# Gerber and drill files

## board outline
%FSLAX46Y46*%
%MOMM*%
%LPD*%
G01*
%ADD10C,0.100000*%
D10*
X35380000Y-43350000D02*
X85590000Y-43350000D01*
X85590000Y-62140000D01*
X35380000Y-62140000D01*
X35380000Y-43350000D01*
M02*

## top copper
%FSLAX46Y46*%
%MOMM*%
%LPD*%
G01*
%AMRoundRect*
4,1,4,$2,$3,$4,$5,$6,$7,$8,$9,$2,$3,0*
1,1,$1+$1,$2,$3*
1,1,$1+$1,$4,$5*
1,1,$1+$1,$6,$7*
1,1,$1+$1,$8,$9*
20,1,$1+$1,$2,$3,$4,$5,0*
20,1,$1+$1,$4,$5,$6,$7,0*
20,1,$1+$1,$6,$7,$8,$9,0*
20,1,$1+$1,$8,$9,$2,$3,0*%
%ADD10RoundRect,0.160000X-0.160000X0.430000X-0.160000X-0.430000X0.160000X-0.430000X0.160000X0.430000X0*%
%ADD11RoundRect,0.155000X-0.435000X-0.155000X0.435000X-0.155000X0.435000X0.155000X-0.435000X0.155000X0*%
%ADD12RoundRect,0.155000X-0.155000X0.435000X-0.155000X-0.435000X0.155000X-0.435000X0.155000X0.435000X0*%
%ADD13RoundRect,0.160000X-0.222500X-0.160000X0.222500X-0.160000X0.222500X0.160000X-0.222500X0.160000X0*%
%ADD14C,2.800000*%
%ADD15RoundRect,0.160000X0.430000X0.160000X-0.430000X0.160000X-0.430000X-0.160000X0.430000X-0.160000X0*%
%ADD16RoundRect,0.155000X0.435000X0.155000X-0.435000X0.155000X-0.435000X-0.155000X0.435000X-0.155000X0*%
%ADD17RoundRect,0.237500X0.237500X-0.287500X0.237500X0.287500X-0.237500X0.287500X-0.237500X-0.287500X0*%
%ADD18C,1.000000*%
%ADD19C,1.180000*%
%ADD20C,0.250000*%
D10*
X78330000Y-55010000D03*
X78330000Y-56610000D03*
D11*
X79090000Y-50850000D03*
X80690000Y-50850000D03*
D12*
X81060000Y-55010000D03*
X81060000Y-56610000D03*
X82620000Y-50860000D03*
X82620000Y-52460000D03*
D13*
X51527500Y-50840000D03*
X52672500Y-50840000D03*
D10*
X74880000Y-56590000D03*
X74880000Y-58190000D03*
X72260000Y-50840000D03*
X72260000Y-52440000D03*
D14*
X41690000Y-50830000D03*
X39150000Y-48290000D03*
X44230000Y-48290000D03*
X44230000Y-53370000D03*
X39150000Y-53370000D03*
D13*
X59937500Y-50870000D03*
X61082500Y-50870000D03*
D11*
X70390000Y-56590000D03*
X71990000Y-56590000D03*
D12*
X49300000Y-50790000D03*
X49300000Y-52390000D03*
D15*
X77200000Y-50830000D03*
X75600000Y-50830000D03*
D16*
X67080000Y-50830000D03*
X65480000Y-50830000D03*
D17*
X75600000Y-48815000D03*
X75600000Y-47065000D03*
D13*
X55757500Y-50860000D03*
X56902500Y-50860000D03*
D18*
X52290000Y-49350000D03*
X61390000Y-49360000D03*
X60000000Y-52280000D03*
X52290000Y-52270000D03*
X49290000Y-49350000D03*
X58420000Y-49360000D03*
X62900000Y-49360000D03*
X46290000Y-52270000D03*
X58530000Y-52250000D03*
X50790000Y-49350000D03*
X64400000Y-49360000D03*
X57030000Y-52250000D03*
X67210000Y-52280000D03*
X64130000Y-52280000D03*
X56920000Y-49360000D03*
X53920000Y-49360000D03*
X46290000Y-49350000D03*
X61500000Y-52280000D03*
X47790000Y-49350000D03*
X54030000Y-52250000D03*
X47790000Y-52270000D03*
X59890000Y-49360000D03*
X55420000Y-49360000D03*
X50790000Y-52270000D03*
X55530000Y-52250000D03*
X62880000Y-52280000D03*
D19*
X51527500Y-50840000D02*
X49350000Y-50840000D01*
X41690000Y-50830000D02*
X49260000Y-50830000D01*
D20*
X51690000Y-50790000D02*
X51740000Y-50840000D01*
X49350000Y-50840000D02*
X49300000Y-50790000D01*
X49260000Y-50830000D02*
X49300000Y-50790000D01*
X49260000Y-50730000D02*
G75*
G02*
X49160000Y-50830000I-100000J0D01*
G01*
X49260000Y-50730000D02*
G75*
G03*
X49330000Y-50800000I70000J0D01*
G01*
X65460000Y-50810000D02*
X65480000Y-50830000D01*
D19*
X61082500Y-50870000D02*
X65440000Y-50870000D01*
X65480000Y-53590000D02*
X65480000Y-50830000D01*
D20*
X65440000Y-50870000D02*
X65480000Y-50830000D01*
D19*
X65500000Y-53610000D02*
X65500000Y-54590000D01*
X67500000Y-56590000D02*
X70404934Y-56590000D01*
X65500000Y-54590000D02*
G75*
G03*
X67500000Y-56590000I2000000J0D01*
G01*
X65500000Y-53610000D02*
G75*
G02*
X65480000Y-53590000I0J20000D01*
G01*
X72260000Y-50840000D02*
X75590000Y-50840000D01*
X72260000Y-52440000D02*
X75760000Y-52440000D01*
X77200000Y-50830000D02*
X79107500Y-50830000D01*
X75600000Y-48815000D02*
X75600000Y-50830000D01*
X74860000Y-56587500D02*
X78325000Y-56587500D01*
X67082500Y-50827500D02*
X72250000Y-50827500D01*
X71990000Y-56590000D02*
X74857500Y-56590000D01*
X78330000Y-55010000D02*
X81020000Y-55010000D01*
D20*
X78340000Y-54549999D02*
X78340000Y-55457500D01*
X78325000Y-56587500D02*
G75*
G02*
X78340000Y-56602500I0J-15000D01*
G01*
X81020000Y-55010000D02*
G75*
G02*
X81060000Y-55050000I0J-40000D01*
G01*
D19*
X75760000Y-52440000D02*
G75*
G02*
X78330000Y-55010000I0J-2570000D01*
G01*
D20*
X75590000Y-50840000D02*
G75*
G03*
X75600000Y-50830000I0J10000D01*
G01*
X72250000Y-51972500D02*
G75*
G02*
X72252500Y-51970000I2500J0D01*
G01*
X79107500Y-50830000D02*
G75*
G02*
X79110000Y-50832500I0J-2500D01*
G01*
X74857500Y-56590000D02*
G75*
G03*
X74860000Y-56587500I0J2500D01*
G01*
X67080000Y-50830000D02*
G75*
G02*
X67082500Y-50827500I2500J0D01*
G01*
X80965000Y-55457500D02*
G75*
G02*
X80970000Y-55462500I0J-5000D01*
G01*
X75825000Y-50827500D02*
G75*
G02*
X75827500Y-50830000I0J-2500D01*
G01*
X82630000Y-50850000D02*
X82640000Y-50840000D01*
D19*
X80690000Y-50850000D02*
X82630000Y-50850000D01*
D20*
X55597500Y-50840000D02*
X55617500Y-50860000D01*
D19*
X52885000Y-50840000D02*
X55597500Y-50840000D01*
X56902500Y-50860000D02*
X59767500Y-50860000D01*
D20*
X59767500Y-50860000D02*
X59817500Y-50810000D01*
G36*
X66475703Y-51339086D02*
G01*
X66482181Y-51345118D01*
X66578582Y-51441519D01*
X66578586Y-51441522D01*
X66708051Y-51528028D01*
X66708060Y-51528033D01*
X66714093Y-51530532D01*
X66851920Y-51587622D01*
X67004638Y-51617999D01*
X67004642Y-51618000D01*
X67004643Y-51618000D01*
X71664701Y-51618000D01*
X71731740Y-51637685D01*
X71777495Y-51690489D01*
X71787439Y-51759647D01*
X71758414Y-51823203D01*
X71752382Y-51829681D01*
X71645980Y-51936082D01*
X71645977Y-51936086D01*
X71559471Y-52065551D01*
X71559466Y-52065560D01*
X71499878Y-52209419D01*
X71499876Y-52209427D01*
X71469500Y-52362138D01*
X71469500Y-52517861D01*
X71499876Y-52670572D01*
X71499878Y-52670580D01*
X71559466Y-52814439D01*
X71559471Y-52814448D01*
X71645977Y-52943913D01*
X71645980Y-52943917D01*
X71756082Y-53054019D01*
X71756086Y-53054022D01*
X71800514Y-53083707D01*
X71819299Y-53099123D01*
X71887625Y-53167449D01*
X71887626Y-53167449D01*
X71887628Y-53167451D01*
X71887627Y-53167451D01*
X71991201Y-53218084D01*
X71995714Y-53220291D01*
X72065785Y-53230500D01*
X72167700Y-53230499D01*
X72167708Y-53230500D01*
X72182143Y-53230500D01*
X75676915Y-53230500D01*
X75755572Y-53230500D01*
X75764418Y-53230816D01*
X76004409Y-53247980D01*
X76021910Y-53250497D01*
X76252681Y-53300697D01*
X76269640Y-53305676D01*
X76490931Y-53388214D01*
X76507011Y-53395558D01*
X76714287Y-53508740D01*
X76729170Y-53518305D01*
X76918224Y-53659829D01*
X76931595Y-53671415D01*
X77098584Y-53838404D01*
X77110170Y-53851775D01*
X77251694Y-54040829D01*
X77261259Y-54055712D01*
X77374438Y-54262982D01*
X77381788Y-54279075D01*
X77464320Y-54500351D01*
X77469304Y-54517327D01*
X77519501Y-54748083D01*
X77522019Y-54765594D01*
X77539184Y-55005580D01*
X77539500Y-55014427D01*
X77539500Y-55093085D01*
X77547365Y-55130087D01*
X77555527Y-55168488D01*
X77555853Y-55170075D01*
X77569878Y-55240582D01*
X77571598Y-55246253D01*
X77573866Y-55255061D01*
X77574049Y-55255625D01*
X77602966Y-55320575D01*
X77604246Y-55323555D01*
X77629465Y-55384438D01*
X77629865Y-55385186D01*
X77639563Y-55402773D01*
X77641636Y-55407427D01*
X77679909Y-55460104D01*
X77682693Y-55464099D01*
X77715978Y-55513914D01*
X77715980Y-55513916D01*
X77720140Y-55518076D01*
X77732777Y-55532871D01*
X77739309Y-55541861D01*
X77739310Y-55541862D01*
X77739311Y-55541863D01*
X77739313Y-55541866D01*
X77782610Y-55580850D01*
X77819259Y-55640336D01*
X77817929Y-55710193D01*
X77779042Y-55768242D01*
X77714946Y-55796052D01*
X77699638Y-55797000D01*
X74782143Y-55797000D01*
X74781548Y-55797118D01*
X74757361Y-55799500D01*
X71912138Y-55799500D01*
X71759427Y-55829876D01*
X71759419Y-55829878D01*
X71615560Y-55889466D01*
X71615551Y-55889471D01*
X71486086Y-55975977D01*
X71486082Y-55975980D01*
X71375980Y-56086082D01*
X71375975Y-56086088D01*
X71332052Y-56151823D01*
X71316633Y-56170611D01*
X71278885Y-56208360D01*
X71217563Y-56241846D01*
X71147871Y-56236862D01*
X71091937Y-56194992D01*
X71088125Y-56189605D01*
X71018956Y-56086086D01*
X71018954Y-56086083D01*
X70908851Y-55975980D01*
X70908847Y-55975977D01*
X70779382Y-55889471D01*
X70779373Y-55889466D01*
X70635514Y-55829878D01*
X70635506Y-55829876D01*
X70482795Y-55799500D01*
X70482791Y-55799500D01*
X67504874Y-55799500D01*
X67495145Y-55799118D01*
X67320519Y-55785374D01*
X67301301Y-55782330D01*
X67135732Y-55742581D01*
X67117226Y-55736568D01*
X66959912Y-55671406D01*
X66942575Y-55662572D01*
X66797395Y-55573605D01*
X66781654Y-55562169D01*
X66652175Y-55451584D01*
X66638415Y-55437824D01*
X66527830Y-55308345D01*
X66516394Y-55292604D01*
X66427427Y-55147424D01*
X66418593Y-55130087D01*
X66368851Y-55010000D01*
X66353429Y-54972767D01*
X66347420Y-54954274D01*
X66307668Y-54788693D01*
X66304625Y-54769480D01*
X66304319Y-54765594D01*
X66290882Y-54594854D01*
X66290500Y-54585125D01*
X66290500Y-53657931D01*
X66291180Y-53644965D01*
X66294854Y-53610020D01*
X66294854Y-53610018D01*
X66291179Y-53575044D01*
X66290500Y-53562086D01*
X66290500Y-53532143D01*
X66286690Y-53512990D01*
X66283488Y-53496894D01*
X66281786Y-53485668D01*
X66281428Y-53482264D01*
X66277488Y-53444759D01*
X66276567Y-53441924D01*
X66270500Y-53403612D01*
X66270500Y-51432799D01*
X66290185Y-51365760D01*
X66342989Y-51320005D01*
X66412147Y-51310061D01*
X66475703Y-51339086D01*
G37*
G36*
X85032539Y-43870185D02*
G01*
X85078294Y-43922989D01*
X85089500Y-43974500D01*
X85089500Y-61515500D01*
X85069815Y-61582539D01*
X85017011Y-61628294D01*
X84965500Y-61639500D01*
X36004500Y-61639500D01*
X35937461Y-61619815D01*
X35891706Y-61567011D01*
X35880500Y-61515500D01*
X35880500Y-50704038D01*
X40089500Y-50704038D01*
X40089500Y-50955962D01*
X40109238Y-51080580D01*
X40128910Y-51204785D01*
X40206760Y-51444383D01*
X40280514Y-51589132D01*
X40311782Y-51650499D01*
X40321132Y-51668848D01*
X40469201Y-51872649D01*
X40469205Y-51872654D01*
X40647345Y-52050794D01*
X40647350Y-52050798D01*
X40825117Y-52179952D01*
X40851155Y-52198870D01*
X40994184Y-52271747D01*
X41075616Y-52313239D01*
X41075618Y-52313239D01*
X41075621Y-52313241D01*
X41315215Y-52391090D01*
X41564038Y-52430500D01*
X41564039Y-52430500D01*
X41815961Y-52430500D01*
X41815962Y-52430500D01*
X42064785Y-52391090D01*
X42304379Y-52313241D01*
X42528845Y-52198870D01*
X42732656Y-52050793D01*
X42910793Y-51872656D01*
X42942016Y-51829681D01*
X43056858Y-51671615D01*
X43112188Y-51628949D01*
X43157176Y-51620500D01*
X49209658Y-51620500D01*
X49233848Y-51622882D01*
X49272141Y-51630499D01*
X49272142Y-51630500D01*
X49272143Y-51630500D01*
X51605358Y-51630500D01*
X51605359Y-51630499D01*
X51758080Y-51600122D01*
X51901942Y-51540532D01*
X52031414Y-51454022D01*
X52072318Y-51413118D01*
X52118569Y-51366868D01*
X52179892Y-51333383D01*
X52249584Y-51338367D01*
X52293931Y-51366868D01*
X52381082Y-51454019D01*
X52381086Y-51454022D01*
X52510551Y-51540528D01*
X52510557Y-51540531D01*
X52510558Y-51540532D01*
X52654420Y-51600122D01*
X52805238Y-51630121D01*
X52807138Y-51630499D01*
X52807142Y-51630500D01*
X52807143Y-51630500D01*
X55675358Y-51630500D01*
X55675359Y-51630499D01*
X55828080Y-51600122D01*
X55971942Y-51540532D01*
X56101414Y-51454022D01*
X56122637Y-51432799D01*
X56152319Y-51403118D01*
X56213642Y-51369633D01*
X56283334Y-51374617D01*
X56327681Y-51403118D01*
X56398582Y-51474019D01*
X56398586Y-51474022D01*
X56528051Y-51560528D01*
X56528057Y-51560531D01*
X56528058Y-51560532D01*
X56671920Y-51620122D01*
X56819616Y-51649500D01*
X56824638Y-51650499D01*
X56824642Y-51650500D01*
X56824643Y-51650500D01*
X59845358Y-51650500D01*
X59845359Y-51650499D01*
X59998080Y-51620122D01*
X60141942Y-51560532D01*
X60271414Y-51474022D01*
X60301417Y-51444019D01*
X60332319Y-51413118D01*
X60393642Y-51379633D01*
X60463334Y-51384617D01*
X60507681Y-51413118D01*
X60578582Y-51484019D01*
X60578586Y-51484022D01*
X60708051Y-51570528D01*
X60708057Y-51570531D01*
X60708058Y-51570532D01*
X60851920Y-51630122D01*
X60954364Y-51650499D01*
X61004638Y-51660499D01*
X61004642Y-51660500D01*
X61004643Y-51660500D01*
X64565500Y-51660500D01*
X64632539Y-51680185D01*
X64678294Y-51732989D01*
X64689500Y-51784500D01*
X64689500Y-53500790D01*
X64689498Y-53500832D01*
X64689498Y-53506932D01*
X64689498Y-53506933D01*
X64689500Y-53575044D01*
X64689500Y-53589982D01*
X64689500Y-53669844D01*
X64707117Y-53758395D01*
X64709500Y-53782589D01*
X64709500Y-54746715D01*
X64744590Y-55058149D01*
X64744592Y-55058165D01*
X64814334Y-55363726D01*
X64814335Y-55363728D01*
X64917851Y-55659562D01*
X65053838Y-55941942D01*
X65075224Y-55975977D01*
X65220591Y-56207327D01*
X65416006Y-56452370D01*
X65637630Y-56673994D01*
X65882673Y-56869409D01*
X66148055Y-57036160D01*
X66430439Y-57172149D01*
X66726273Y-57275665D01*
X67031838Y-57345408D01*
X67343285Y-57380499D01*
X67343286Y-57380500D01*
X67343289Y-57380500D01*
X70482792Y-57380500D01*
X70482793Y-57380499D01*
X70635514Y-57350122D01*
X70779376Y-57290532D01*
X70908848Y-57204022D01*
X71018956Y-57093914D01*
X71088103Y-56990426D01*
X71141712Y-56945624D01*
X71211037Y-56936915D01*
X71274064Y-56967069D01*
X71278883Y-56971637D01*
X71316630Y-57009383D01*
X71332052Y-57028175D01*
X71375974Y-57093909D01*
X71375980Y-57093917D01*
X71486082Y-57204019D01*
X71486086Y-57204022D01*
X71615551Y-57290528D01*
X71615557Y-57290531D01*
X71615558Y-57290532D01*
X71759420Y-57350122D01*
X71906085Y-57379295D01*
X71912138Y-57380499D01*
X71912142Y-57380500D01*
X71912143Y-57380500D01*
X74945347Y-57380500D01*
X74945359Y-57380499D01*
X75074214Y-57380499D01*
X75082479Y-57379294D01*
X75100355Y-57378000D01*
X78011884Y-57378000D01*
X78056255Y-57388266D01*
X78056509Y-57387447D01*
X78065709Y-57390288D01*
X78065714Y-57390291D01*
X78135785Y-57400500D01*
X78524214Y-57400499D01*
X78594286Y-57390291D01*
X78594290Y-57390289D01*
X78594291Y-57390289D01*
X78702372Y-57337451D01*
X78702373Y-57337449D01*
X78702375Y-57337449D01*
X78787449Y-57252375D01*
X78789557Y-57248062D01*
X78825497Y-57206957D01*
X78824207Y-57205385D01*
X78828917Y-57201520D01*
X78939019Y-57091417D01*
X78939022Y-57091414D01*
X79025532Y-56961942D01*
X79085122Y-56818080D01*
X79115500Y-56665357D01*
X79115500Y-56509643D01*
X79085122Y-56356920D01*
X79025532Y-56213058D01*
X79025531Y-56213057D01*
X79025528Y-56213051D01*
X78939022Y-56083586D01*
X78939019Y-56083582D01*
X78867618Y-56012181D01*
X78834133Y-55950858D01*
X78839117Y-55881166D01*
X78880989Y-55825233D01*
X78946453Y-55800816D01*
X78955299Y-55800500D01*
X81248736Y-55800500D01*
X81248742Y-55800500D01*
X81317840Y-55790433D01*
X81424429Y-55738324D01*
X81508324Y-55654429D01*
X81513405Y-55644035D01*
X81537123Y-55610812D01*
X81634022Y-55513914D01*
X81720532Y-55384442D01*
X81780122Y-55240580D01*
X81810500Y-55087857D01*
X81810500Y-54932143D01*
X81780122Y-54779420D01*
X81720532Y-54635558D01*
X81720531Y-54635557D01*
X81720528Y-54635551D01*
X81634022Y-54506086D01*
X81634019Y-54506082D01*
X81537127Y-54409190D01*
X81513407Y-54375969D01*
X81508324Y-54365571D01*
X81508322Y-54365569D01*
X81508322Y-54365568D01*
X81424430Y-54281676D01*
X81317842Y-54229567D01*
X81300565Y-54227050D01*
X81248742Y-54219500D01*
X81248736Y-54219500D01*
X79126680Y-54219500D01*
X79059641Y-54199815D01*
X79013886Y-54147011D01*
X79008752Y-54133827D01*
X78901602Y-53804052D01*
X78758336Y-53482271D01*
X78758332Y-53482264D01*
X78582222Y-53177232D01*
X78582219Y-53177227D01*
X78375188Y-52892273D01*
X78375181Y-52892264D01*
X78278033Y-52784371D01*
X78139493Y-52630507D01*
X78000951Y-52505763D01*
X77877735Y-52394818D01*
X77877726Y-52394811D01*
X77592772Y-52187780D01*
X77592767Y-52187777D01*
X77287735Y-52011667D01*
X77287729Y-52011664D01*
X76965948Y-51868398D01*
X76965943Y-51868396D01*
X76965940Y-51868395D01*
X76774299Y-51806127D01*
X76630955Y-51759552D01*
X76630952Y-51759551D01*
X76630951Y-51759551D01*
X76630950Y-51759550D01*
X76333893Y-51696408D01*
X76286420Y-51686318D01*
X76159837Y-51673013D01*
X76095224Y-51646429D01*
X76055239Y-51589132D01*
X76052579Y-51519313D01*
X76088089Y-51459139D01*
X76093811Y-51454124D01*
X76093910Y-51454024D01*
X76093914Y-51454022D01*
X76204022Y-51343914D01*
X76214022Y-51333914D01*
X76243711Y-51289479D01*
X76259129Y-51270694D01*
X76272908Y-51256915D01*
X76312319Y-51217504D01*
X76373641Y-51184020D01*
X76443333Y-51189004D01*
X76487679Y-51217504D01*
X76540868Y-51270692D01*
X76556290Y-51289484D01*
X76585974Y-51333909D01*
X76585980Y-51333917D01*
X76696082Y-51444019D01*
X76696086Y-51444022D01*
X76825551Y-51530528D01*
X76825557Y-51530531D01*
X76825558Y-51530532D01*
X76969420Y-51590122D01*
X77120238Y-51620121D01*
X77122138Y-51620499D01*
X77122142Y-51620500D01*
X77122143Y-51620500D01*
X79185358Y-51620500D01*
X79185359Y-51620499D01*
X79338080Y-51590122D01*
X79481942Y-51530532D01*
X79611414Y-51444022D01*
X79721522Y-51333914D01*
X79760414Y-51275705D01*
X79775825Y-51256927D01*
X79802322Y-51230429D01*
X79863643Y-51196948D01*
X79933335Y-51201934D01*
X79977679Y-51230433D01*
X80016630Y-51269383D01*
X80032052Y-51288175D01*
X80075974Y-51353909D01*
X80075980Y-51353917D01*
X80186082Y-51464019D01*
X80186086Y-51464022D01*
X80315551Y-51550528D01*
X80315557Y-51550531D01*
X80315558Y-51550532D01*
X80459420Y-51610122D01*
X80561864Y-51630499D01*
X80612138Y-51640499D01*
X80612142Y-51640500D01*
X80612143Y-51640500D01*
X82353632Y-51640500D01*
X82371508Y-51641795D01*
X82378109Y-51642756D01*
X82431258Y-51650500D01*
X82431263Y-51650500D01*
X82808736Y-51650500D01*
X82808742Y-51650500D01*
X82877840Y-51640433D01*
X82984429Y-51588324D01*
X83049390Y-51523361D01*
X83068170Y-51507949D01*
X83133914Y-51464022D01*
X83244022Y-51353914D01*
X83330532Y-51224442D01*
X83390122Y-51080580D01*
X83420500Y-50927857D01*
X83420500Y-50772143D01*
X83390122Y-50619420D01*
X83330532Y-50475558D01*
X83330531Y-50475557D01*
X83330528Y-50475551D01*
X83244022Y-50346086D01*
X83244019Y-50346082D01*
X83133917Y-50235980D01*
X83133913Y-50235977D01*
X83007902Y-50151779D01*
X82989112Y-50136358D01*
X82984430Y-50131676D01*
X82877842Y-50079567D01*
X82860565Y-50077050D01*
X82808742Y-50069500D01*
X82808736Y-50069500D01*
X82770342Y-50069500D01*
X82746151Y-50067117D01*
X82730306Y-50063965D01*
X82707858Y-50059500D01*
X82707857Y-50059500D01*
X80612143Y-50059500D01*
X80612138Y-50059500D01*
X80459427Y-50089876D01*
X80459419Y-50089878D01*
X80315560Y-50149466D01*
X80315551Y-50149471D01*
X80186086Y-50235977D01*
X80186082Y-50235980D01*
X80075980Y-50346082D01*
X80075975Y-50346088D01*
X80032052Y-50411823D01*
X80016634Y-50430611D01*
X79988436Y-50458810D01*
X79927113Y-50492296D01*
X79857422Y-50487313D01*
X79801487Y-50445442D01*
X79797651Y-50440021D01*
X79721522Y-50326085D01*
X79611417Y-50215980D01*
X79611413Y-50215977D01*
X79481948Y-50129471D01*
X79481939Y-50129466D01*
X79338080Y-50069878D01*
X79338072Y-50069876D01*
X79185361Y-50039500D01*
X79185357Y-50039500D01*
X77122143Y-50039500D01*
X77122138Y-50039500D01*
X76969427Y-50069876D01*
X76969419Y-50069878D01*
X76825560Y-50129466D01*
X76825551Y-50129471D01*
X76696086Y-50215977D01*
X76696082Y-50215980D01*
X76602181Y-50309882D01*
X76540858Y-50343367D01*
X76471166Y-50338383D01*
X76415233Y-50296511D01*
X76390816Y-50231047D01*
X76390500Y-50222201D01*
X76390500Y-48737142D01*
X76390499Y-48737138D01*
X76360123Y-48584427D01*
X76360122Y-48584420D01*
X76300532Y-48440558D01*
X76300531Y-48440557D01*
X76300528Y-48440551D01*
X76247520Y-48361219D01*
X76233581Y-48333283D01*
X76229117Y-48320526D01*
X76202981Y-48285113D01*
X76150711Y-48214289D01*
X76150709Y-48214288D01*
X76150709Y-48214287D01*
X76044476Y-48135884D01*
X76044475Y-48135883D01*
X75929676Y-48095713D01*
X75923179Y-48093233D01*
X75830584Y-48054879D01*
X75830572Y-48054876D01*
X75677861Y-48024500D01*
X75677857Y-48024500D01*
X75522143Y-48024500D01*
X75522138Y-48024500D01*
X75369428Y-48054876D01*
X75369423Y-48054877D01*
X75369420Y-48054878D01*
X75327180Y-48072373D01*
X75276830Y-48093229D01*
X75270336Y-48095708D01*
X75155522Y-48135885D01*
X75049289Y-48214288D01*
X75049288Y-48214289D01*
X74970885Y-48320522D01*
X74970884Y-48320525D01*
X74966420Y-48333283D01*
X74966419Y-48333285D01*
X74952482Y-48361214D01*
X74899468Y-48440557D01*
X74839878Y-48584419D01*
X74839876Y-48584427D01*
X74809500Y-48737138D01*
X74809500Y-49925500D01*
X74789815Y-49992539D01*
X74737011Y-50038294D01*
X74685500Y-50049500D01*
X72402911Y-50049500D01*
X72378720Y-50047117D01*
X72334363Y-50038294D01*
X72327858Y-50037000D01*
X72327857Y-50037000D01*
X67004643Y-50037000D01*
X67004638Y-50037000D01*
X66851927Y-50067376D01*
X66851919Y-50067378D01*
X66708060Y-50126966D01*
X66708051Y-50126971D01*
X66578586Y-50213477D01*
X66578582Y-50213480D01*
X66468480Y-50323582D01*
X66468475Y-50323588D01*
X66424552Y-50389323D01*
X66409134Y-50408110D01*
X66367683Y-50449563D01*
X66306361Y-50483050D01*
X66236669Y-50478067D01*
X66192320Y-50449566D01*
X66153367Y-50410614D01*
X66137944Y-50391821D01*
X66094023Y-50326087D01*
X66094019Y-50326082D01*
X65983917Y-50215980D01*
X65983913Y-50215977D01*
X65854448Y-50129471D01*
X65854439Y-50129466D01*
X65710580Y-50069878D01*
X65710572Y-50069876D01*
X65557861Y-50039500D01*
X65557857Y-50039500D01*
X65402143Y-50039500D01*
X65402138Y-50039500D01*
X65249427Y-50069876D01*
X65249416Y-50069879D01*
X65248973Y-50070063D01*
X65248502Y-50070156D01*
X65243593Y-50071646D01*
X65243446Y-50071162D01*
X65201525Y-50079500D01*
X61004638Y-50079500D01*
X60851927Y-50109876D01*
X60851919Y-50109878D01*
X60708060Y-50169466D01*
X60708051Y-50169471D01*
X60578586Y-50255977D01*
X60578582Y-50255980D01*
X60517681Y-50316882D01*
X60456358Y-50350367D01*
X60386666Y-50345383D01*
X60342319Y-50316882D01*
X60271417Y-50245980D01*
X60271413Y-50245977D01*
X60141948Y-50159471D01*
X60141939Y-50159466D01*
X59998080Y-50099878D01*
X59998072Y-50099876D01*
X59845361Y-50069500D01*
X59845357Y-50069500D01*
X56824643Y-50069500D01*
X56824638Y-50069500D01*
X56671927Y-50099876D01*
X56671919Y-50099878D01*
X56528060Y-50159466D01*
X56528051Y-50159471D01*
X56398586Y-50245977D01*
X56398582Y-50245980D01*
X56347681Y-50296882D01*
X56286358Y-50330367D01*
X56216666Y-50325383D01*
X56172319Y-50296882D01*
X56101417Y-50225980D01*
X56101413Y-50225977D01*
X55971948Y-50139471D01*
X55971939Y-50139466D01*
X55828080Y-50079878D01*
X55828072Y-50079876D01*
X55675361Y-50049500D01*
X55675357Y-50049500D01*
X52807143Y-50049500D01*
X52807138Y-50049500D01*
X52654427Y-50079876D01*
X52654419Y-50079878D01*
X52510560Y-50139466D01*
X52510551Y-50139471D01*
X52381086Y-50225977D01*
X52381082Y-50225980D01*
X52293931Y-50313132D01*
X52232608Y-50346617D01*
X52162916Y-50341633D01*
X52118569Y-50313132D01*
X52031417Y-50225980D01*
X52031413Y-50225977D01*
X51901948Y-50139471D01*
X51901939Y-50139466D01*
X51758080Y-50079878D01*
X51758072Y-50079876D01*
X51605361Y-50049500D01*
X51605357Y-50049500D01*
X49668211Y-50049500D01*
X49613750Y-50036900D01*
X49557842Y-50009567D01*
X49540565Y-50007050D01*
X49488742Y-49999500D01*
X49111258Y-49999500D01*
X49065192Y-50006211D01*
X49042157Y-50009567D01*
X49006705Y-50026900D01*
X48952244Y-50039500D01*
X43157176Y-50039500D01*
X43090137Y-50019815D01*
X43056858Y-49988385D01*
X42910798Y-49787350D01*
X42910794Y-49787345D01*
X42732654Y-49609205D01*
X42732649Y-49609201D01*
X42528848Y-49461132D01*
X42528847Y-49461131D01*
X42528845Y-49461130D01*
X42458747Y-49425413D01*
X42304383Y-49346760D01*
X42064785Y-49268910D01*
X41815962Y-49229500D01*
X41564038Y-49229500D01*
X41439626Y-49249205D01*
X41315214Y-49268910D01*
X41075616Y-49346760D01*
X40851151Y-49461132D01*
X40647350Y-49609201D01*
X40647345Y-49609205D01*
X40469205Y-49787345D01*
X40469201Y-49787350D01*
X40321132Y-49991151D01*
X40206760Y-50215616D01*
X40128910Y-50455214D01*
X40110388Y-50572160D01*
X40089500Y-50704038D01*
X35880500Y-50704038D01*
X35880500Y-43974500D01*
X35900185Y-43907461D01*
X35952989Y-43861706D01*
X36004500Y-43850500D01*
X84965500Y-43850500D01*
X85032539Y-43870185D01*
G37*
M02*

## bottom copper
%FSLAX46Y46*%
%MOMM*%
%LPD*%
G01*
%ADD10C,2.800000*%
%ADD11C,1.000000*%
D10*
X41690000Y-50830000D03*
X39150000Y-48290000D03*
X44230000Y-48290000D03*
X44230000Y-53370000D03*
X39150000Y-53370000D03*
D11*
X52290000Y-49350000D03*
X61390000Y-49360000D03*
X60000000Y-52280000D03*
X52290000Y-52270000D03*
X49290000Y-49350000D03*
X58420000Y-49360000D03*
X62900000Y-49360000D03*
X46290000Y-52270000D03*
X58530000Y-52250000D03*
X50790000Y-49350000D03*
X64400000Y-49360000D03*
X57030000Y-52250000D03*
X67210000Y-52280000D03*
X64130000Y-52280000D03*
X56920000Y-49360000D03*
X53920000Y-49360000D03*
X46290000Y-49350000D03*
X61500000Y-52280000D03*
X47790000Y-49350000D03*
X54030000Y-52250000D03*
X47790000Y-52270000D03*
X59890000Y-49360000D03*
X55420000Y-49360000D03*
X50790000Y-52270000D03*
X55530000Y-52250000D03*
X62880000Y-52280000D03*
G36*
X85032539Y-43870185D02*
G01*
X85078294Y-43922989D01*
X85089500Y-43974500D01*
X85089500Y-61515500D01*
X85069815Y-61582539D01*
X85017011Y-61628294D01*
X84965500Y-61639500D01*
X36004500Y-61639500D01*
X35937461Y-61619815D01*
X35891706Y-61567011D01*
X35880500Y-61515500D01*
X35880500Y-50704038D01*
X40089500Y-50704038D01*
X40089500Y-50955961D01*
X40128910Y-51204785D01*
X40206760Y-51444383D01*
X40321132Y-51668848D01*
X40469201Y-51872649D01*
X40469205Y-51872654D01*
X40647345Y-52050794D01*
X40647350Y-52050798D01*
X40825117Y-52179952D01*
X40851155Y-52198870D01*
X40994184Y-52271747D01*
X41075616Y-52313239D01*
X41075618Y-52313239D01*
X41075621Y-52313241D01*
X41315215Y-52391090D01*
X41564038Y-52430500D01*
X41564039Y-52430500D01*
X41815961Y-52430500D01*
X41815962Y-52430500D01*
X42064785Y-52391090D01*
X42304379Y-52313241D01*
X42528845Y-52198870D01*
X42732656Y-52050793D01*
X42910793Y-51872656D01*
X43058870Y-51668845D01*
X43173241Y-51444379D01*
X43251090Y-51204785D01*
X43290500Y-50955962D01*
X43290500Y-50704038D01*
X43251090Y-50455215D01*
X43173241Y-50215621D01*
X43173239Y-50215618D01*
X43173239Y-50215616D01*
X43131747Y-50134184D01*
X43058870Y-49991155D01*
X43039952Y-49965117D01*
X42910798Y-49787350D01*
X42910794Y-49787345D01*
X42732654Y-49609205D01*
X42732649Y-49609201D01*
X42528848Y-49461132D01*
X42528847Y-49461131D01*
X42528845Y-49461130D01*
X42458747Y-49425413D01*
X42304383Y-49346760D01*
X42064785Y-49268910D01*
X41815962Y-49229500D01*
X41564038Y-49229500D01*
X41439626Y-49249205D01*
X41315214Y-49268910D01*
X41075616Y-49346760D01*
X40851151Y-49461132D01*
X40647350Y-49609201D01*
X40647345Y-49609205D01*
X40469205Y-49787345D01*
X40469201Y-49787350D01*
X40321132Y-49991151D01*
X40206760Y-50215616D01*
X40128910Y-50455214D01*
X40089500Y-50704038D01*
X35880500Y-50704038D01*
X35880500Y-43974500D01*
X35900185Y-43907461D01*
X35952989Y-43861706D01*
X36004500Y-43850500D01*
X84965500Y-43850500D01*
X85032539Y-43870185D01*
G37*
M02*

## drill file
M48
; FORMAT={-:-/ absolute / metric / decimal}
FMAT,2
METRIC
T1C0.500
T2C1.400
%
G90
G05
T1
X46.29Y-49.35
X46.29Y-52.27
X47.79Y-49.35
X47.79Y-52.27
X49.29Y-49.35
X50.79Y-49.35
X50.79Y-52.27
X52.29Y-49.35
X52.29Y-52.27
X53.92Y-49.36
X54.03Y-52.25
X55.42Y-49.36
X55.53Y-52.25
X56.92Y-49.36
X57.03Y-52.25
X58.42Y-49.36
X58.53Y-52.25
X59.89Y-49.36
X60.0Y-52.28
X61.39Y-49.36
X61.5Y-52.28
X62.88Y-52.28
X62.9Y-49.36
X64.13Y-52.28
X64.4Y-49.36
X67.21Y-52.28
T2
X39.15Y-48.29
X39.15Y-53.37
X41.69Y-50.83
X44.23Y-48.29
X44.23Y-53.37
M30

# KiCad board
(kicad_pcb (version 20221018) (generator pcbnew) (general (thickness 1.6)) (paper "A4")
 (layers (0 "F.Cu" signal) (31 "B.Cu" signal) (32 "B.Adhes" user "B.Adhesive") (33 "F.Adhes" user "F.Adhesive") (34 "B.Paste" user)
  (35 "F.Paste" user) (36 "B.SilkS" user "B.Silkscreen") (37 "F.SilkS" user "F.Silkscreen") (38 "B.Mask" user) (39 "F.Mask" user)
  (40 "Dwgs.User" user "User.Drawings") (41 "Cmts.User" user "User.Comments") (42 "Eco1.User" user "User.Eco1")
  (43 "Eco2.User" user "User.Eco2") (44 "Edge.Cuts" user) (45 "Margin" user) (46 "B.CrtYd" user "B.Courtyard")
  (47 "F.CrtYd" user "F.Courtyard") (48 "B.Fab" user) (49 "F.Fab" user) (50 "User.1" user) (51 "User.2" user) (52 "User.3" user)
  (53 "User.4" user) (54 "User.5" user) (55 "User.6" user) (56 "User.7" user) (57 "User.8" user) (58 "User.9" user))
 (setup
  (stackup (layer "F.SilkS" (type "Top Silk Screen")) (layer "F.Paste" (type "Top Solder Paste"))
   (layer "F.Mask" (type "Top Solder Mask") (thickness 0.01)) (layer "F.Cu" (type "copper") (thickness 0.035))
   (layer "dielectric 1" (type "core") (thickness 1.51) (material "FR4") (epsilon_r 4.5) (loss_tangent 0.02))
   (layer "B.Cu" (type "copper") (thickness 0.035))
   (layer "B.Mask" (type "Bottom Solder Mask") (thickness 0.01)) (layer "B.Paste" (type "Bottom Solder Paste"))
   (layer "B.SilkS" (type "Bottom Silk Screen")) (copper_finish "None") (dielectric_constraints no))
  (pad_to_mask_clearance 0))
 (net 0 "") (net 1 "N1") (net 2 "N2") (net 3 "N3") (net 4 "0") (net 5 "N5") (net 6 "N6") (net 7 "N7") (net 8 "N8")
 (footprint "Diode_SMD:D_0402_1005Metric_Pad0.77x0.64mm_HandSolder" (layer "F.Cu") (at 78.33 55.81 -90)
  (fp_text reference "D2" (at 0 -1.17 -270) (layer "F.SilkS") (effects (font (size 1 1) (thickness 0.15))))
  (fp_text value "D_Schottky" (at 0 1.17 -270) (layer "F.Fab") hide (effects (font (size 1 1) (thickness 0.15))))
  (pad "1" smd roundrect (at -0.8 0 270) (size 1.18 0.64) (layers "F.Cu" "F.Paste" "F.Mask") (roundrect_rratio 0.25) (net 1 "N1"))
  (pad "2" smd roundrect (at 0.8 0 270) (size 1.18 0.64) (layers "F.Cu" "F.Paste" "F.Mask") (roundrect_rratio 0.25) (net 1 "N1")))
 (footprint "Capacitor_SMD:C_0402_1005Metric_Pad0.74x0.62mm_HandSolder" (layer "F.Cu") (at 79.89 50.85)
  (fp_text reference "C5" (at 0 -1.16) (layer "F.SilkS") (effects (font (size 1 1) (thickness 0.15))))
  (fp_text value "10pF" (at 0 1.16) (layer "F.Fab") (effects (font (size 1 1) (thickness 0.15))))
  (pad "1" smd roundrect (at -0.8 0) (size 1.18 0.62) (layers "F.Cu" "F.Paste" "F.Mask") (roundrect_rratio 0.25) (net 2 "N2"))
  (pad "2" smd roundrect (at 0.8 0) (size 1.18 0.62) (layers "F.Cu" "F.Paste" "F.Mask") (roundrect_rratio 0.25) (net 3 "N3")))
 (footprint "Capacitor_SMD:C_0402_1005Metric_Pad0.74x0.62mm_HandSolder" (layer "F.Cu") (at 81.06 55.81 -90)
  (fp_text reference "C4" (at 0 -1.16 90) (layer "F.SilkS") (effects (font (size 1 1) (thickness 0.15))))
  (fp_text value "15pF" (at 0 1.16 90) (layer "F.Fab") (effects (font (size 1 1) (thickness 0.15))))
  (pad "1" smd roundrect (at -0.8 0 270) (size 1.18 0.62) (layers "F.Cu" "F.Paste" "F.Mask") (roundrect_rratio 0.25) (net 1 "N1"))
  (pad "2" smd roundrect (at 0.8 0 270) (size 1.18 0.62) (layers "F.Cu" "F.Paste" "F.Mask") (roundrect_rratio 0.25) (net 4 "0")))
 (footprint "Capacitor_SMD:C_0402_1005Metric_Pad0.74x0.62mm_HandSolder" (layer "F.Cu") (at 82.62 51.66 -90)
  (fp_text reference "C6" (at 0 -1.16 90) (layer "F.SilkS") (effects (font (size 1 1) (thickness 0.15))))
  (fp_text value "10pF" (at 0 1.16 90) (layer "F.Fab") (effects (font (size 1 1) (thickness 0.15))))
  (pad "1" smd roundrect (at -0.8 0 270) (size 1.18 0.62) (layers "F.Cu" "F.Paste" "F.Mask") (roundrect_rratio 0.25) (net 3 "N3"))
  (pad "2" smd roundrect (at 0.8 0 270) (size 1.18 0.62) (layers "F.Cu" "F.Paste" "F.Mask") (roundrect_rratio 0.25) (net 4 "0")))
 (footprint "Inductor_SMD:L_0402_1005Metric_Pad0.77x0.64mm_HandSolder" (layer "F.Cu") (at 52.1 50.84)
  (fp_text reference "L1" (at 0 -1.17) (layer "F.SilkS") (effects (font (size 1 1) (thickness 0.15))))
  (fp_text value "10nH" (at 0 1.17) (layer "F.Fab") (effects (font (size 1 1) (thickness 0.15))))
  (pad "1" smd roundrect (at -0.5725 0) (size 0.765 0.64) (layers "F.Cu" "F.Paste" "F.Mask") (roundrect_rratio 0.25) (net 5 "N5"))
  (pad "2" smd roundrect (at 0.5725 0) (size 0.765 0.64) (layers "F.Cu" "F.Paste" "F.Mask") (roundrect_rratio 0.25) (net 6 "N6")))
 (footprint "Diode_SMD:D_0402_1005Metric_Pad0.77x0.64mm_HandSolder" (layer "F.Cu") (at 74.88 57.39 -90)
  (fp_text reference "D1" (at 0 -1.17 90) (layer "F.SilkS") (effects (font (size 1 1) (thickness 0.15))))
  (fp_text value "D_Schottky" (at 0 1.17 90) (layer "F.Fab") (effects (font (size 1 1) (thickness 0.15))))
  (pad "1" smd roundrect (at -0.8 0 270) (size 1.18 0.64) (layers "F.Cu" "F.Paste" "F.Mask") (roundrect_rratio 0.25) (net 1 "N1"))
  (pad "2" smd roundrect (at 0.8 0 270) (size 1.18 0.64) (layers "F.Cu" "F.Paste" "F.Mask") (roundrect_rratio 0.25) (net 4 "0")))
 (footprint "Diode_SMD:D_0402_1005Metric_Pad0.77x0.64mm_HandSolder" (layer "F.Cu") (at 72.26 51.64 -90)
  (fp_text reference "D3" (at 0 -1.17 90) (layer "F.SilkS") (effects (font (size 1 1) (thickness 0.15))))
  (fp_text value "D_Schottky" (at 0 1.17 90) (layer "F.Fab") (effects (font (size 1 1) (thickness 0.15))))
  (pad "1" smd roundrect (at -0.8 0 270) (size 1.18 0.64) (layers "F.Cu" "F.Paste" "F.Mask") (roundrect_rratio 0.25) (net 1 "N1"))
  (pad "2" smd roundrect (at 0.8 0 270) (size 1.18 0.64) (layers "F.Cu" "F.Paste" "F.Mask") (roundrect_rratio 0.25) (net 1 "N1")))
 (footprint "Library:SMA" (layer "F.Cu") (at 41.69 50.83)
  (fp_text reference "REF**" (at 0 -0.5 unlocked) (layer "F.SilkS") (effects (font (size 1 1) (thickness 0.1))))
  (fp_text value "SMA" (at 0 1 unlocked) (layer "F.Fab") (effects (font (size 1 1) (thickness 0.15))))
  (pad "1" thru_hole circle (at 0 0) (size 2.8 2.8) (drill 1.4) (layers "*.Cu" "*.Mask") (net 5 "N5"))
  (pad "2" thru_hole circle (at -2.54 -2.54) (size 2.8 2.8) (drill 1.4) (layers "*.Cu" "*.Mask") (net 4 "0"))
  (pad "3" thru_hole circle (at 2.54 -2.54) (size 2.8 2.8) (drill 1.4) (layers "*.Cu" "*.Mask") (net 4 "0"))
  (pad "4" thru_hole circle (at 2.54 2.54) (size 2.8 2.8) (drill 1.4) (layers "*.Cu" "*.Mask") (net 4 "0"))
  (pad "5" thru_hole circle (at -2.54 2.54) (size 2.8 2.8) (drill 1.4) (layers "*.Cu" "*.Mask") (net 4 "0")))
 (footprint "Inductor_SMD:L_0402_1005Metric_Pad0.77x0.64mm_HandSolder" (layer "F.Cu") (at 60.51 50.87)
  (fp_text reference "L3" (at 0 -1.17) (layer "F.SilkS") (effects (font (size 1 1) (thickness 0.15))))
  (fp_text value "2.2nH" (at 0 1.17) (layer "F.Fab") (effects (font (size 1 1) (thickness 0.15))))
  (pad "1" smd roundrect (at -0.5725 0) (size 0.765 0.64) (layers "F.Cu" "F.Paste" "F.Mask") (roundrect_rratio 0.25) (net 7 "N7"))
  (pad "2" smd roundrect (at 0.5725 0) (size 0.765 0.64) (layers "F.Cu" "F.Paste" "F.Mask") (roundrect_rratio 0.25) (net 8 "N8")))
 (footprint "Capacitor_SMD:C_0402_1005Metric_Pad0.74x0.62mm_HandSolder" (layer "F.Cu") (at 71.19 56.59)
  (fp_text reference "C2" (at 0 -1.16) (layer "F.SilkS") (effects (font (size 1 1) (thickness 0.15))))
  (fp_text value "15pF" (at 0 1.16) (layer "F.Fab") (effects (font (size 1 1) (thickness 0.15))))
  (pad "1" smd roundrect (at -0.8 0) (size 1.18 0.62) (layers "F.Cu" "F.Paste" "F.Mask") (roundrect_rratio 0.25) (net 8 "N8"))
  (pad "2" smd roundrect (at 0.8 0) (size 1.18 0.62) (layers "F.Cu" "F.Paste" "F.Mask") (roundrect_rratio 0.25) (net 1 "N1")))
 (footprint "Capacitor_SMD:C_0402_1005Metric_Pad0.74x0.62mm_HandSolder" (layer "F.Cu") (at 49.3 51.59 -90)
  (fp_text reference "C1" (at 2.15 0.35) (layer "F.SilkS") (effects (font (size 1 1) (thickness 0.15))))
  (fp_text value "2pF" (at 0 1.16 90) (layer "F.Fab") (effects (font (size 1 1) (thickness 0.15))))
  (pad "1" smd roundrect (at -0.8 0 270) (size 1.18 0.62) (layers "F.Cu" "F.Paste" "F.Mask") (roundrect_rratio 0.25) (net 5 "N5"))
  (pad "2" smd roundrect (at 0.8 0 270) (size 1.18 0.62) (layers "F.Cu" "F.Paste" "F.Mask") (roundrect_rratio 0.25) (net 4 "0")))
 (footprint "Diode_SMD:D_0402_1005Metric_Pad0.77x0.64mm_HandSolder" (layer "F.Cu") (at 76.4 50.83 180)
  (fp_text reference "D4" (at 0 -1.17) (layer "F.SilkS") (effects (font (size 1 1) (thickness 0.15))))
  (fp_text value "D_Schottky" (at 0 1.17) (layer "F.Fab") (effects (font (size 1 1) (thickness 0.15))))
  (pad "1" smd roundrect (at -0.8 0 180) (size 1.18 0.64) (layers "F.Cu" "F.Paste" "F.Mask") (roundrect_rratio 0.25) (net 1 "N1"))
  (pad "2" smd roundrect (at 0.8 0 180) (size 1.18 0.64) (layers "F.Cu" "F.Paste" "F.Mask") (roundrect_rratio 0.25) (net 1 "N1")))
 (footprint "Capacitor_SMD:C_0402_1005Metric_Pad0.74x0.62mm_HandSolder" (layer "F.Cu") (at 66.28 50.83 180)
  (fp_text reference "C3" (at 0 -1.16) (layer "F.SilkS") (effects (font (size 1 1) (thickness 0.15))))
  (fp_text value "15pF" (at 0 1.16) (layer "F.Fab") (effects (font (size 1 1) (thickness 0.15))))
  (pad "1" smd roundrect (at -0.8 0 180) (size 1.18 0.62) (layers "F.Cu" "F.Paste" "F.Mask") (roundrect_rratio 0.25) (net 1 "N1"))
  (pad "2" smd roundrect (at 0.8 0 180) (size 1.18 0.62) (layers "F.Cu" "F.Paste" "F.Mask") (roundrect_rratio 0.25) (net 8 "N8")))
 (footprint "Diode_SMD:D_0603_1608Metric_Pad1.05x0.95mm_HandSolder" (layer "F.Cu") (at 75.6 47.94 90)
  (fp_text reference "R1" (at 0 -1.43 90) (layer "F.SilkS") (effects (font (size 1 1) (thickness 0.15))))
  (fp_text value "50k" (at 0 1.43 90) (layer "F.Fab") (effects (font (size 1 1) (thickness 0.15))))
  (pad "1" smd roundrect (at -0.875 0 90) (size 1.05 0.95) (layers "F.Cu" "F.Paste" "F.Mask") (roundrect_rratio 0.25) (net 1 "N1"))
  (pad "2" smd roundrect (at 0.875 0 90) (size 1.05 0.95) (layers "F.Cu" "F.Paste" "F.Mask") (roundrect_rratio 0.25) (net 4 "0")))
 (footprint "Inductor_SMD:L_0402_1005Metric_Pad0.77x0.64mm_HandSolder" (layer "F.Cu") (at 56.33 50.86)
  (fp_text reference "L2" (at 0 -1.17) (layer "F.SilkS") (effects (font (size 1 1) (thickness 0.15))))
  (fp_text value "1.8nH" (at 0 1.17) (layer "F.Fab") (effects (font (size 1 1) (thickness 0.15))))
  (pad "1" smd roundrect (at -0.5725 0) (size 0.765 0.64) (layers "F.Cu" "F.Paste" "F.Mask") (roundrect_rratio 0.25) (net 6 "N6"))
  (pad "2" smd roundrect (at 0.5725 0) (size 0.765 0.64) (layers "F.Cu" "F.Paste" "F.Mask") (roundrect_rratio 0.25) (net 7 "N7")))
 (gr_rect (start 35.38 43.35) (end 85.59 62.14) (stroke (width 0.1) (type default)) (fill none) (layer "Edge.Cuts"))
 (segment (start 51.5275 50.84) (end 49.35 50.84) (width 1.18) (layer "F.Cu") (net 5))
 (segment (start 41.69 50.83) (end 49.26 50.83) (width 1.18) (layer "F.Cu") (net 5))
 (segment (start 51.69 50.79) (end 51.74 50.84) (width 0.25) (layer "F.Cu") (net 5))
 (segment (start 49.35 50.84) (end 49.3 50.79) (width 0.25) (layer "F.Cu") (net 5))
 (segment (start 49.26 50.83) (end 49.3 50.79) (width 0.25) (layer "F.Cu") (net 5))
 (arc (start 49.26 50.73) (mid 49.230711 50.800711) (end 49.16 50.83) (width 0.25) (layer "F.Cu") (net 5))
 (arc (start 49.26 50.73) (mid 49.280503 50.779497) (end 49.33 50.8) (width 0.25) (layer "F.Cu") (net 5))
 (via (at 52.29 49.35) (size 1) (drill 0.5) (layers "F.Cu" "B.Cu") (free) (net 4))
 (via (at 61.39 49.36) (size 1) (drill 0.5) (layers "F.Cu" "B.Cu") (free) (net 4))
 (via (at 60 52.28) (size 1) (drill 0.5) (layers "F.Cu" "B.Cu") (free) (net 4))
 (via (at 52.29 52.27) (size 1) (drill 0.5) (layers "F.Cu" "B.Cu") (free) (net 4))
 (via (at 49.29 49.35) (size 1) (drill 0.5) (layers "F.Cu" "B.Cu") (free) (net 4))
 (via (at 58.42 49.36) (size 1) (drill 0.5) (layers "F.Cu" "B.Cu") (free) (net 4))
 (via (at 62.9 49.36) (size 1) (drill 0.5) (layers "F.Cu" "B.Cu") (free) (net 4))
 (via (at 46.29 52.27) (size 1) (drill 0.5) (layers "F.Cu" "B.Cu") (free) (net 4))
 (via (at 58.53 52.25) (size 1) (drill 0.5) (layers "F.Cu" "B.Cu") (free) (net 4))
 (via (at 50.79 49.35) (size 1) (drill 0.5) (layers "F.Cu" "B.Cu") (free) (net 4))
 (via (at 64.4 49.36) (size 1) (drill 0.5) (layers "F.Cu" "B.Cu") (free) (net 4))
 (via (at 57.03 52.25) (size 1) (drill 0.5) (layers "F.Cu" "B.Cu") (free) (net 4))
 (via (at 67.21 52.28) (size 1) (drill 0.5) (layers "F.Cu" "B.Cu") (free) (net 4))
 (via (at 64.13 52.28) (size 1) (drill 0.5) (layers "F.Cu" "B.Cu") (free) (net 4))
 (via (at 56.92 49.36) (size 1) (drill 0.5) (layers "F.Cu" "B.Cu") (free) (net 4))
 (via (at 53.92 49.36) (size 1) (drill 0.5) (layers "F.Cu" "B.Cu") (free) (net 4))
 (via (at 46.29 49.35) (size 1) (drill 0.5) (layers "F.Cu" "B.Cu") (free) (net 4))
 (via (at 61.5 52.28) (size 1) (drill 0.5) (layers "F.Cu" "B.Cu") (free) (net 4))
 (via (at 47.79 49.35) (size 1) (drill 0.5) (layers "F.Cu" "B.Cu") (free) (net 4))
 (via (at 54.03 52.25) (size 1) (drill 0.5) (layers "F.Cu" "B.Cu") (free) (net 4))
 (via (at 47.79 52.27) (size 1) (drill 0.5) (layers "F.Cu" "B.Cu") (free) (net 4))
 (via (at 59.89 49.36) (size 1) (drill 0.5) (layers "F.Cu" "B.Cu") (free) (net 4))
 (via (at 55.42 49.36) (size 1) (drill 0.5) (layers "F.Cu" "B.Cu") (free) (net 4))
 (via (at 50.79 52.27) (size 1) (drill 0.5) (layers "F.Cu" "B.Cu") (free) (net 4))
 (via (at 55.53 52.25) (size 1) (drill 0.5) (layers "F.Cu" "B.Cu") (free) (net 4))
 (via (at 62.88 52.28) (size 1) (drill 0.5) (layers "F.Cu" "B.Cu") (free) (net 4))
 (segment (start 65.46 50.81) (end 65.48 50.83) (width 0.25) (layer "F.Cu") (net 8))
 (segment (start 61.0825 50.87) (end 65.44 50.87) (width 1.18) (layer "F.Cu") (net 8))
 (segment (start 65.48 53.59) (end 65.48 50.83) (width 1.18) (layer "F.Cu") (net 8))
 (segment (start 65.44 50.87) (end 65.48 50.83) (width 0.25) (layer "F.Cu") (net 8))
 (segment (start 65.5 53.61) (end 65.5 54.59) (width 1.18) (layer "F.Cu") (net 8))
 (segment (start 67.5 56.59) (end 70.404934 56.59) (width 1.18) (layer "F.Cu") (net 8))
 (arc (start 65.5 54.59) (mid 66.085786 56.004214) (end 67.5 56.59) (width 1.18) (layer "F.Cu") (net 8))
 (arc (start 65.5 53.61) (mid 65.485858 53.604142) (end 65.48 53.59) (width 1.18) (layer "F.Cu") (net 8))
 (segment (start 72.26 50.84) (end 75.59 50.84) (width 1.18) (layer "F.Cu") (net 1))
 (segment (start 72.26 52.44) (end 75.76 52.44) (width 1.18) (layer "F.Cu") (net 1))
 (segment (start 77.2 50.83) (end 79.1075 50.83) (width 1.18) (layer "F.Cu") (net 1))
 (segment (start 75.6 48.815) (end 75.6 50.83) (width 1.18) (layer "F.Cu") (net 1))
 (segment (start 74.86 56.5875) (end 78.325 56.5875) (width 1.18) (layer "F.Cu") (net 1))
 (segment (start 67.0825 50.8275) (end 72.25 50.8275) (width 1.18) (layer "F.Cu") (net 1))
 (segment (start 71.99 56.59) (end 74.8575 56.59) (width 1.18) (layer "F.Cu") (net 1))
 (segment (start 78.33 55.01) (end 81.02 55.01) (width 1.18) (layer "F.Cu") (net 1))
 (segment (start 78.34 54.549999) (end 78.34 55.4575) (width 0.25) (layer "F.Cu") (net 1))
 (arc (start 78.325 56.5875) (mid 78.335607 56.591893) (end 78.34 56.6025) (width 0.25) (layer "F.Cu") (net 1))
 (arc (start 81.02 55.01) (mid 81.048284 55.021716) (end 81.06 55.05) (width 0.25) (layer "F.Cu") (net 1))
 (arc (start 75.76 52.44) (mid 77.577264 53.192736) (end 78.33 55.01) (width 1.18) (layer "F.Cu") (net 1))
 (arc (start 75.59 50.84) (mid 75.597071 50.837071) (end 75.6 50.83) (width 0.25) (layer "F.Cu") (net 1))
 (arc (start 72.25 51.9725) (mid 72.250732 51.970732) (end 72.2525 51.97) (width 0.25) (layer "F.Cu") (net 1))
 (arc (start 79.1075 50.83) (mid 79.109268 50.830732) (end 79.11 50.8325) (width 0.25) (layer "F.Cu") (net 1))
 (arc (start 74.8575 56.59) (mid 74.859268 56.589268) (end 74.86 56.5875) (width 0.25) (layer "F.Cu") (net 1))
 (arc (start 67.08 50.83) (mid 67.080732 50.828232) (end 67.0825 50.8275) (width 0.25) (layer "F.Cu") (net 1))
 (arc (start 80.965 55.4575) (mid 80.968536 55.458964) (end 80.97 55.4625) (width 0.25) (layer "F.Cu") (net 1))
 (arc (start 75.825 50.8275) (mid 75.826768 50.828232) (end 75.8275 50.83) (width 0.25) (layer "F.Cu") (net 1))
 (segment (start 82.63 50.85) (end 82.64 50.84) (width 0.25) (layer "F.Cu") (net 3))
 (segment (start 80.69 50.85) (end 82.63 50.85) (width 1.18) (layer "F.Cu") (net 3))
 (segment (start 55.5975 50.84) (end 55.6175 50.86) (width 0.25) (layer "F.Cu") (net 6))
 (segment (start 52.885 50.84) (end 55.5975 50.84) (width 1.18) (layer "F.Cu") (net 6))
 (segment (start 56.9025 50.86) (end 59.7675 50.86) (width 1.18) (layer "F.Cu") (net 7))
 (segment (start 59.7675 50.86) (end 59.8175 50.81) (width 0.25) (layer "F.Cu") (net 7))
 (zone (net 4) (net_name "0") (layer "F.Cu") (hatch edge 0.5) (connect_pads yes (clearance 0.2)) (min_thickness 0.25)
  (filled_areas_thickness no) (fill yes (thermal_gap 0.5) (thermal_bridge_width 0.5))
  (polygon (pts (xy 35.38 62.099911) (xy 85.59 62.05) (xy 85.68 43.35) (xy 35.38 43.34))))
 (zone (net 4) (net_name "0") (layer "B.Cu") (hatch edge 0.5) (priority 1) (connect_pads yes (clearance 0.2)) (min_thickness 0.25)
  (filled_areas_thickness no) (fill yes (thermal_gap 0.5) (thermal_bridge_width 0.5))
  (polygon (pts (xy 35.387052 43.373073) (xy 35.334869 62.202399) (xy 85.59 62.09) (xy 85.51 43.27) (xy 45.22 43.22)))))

